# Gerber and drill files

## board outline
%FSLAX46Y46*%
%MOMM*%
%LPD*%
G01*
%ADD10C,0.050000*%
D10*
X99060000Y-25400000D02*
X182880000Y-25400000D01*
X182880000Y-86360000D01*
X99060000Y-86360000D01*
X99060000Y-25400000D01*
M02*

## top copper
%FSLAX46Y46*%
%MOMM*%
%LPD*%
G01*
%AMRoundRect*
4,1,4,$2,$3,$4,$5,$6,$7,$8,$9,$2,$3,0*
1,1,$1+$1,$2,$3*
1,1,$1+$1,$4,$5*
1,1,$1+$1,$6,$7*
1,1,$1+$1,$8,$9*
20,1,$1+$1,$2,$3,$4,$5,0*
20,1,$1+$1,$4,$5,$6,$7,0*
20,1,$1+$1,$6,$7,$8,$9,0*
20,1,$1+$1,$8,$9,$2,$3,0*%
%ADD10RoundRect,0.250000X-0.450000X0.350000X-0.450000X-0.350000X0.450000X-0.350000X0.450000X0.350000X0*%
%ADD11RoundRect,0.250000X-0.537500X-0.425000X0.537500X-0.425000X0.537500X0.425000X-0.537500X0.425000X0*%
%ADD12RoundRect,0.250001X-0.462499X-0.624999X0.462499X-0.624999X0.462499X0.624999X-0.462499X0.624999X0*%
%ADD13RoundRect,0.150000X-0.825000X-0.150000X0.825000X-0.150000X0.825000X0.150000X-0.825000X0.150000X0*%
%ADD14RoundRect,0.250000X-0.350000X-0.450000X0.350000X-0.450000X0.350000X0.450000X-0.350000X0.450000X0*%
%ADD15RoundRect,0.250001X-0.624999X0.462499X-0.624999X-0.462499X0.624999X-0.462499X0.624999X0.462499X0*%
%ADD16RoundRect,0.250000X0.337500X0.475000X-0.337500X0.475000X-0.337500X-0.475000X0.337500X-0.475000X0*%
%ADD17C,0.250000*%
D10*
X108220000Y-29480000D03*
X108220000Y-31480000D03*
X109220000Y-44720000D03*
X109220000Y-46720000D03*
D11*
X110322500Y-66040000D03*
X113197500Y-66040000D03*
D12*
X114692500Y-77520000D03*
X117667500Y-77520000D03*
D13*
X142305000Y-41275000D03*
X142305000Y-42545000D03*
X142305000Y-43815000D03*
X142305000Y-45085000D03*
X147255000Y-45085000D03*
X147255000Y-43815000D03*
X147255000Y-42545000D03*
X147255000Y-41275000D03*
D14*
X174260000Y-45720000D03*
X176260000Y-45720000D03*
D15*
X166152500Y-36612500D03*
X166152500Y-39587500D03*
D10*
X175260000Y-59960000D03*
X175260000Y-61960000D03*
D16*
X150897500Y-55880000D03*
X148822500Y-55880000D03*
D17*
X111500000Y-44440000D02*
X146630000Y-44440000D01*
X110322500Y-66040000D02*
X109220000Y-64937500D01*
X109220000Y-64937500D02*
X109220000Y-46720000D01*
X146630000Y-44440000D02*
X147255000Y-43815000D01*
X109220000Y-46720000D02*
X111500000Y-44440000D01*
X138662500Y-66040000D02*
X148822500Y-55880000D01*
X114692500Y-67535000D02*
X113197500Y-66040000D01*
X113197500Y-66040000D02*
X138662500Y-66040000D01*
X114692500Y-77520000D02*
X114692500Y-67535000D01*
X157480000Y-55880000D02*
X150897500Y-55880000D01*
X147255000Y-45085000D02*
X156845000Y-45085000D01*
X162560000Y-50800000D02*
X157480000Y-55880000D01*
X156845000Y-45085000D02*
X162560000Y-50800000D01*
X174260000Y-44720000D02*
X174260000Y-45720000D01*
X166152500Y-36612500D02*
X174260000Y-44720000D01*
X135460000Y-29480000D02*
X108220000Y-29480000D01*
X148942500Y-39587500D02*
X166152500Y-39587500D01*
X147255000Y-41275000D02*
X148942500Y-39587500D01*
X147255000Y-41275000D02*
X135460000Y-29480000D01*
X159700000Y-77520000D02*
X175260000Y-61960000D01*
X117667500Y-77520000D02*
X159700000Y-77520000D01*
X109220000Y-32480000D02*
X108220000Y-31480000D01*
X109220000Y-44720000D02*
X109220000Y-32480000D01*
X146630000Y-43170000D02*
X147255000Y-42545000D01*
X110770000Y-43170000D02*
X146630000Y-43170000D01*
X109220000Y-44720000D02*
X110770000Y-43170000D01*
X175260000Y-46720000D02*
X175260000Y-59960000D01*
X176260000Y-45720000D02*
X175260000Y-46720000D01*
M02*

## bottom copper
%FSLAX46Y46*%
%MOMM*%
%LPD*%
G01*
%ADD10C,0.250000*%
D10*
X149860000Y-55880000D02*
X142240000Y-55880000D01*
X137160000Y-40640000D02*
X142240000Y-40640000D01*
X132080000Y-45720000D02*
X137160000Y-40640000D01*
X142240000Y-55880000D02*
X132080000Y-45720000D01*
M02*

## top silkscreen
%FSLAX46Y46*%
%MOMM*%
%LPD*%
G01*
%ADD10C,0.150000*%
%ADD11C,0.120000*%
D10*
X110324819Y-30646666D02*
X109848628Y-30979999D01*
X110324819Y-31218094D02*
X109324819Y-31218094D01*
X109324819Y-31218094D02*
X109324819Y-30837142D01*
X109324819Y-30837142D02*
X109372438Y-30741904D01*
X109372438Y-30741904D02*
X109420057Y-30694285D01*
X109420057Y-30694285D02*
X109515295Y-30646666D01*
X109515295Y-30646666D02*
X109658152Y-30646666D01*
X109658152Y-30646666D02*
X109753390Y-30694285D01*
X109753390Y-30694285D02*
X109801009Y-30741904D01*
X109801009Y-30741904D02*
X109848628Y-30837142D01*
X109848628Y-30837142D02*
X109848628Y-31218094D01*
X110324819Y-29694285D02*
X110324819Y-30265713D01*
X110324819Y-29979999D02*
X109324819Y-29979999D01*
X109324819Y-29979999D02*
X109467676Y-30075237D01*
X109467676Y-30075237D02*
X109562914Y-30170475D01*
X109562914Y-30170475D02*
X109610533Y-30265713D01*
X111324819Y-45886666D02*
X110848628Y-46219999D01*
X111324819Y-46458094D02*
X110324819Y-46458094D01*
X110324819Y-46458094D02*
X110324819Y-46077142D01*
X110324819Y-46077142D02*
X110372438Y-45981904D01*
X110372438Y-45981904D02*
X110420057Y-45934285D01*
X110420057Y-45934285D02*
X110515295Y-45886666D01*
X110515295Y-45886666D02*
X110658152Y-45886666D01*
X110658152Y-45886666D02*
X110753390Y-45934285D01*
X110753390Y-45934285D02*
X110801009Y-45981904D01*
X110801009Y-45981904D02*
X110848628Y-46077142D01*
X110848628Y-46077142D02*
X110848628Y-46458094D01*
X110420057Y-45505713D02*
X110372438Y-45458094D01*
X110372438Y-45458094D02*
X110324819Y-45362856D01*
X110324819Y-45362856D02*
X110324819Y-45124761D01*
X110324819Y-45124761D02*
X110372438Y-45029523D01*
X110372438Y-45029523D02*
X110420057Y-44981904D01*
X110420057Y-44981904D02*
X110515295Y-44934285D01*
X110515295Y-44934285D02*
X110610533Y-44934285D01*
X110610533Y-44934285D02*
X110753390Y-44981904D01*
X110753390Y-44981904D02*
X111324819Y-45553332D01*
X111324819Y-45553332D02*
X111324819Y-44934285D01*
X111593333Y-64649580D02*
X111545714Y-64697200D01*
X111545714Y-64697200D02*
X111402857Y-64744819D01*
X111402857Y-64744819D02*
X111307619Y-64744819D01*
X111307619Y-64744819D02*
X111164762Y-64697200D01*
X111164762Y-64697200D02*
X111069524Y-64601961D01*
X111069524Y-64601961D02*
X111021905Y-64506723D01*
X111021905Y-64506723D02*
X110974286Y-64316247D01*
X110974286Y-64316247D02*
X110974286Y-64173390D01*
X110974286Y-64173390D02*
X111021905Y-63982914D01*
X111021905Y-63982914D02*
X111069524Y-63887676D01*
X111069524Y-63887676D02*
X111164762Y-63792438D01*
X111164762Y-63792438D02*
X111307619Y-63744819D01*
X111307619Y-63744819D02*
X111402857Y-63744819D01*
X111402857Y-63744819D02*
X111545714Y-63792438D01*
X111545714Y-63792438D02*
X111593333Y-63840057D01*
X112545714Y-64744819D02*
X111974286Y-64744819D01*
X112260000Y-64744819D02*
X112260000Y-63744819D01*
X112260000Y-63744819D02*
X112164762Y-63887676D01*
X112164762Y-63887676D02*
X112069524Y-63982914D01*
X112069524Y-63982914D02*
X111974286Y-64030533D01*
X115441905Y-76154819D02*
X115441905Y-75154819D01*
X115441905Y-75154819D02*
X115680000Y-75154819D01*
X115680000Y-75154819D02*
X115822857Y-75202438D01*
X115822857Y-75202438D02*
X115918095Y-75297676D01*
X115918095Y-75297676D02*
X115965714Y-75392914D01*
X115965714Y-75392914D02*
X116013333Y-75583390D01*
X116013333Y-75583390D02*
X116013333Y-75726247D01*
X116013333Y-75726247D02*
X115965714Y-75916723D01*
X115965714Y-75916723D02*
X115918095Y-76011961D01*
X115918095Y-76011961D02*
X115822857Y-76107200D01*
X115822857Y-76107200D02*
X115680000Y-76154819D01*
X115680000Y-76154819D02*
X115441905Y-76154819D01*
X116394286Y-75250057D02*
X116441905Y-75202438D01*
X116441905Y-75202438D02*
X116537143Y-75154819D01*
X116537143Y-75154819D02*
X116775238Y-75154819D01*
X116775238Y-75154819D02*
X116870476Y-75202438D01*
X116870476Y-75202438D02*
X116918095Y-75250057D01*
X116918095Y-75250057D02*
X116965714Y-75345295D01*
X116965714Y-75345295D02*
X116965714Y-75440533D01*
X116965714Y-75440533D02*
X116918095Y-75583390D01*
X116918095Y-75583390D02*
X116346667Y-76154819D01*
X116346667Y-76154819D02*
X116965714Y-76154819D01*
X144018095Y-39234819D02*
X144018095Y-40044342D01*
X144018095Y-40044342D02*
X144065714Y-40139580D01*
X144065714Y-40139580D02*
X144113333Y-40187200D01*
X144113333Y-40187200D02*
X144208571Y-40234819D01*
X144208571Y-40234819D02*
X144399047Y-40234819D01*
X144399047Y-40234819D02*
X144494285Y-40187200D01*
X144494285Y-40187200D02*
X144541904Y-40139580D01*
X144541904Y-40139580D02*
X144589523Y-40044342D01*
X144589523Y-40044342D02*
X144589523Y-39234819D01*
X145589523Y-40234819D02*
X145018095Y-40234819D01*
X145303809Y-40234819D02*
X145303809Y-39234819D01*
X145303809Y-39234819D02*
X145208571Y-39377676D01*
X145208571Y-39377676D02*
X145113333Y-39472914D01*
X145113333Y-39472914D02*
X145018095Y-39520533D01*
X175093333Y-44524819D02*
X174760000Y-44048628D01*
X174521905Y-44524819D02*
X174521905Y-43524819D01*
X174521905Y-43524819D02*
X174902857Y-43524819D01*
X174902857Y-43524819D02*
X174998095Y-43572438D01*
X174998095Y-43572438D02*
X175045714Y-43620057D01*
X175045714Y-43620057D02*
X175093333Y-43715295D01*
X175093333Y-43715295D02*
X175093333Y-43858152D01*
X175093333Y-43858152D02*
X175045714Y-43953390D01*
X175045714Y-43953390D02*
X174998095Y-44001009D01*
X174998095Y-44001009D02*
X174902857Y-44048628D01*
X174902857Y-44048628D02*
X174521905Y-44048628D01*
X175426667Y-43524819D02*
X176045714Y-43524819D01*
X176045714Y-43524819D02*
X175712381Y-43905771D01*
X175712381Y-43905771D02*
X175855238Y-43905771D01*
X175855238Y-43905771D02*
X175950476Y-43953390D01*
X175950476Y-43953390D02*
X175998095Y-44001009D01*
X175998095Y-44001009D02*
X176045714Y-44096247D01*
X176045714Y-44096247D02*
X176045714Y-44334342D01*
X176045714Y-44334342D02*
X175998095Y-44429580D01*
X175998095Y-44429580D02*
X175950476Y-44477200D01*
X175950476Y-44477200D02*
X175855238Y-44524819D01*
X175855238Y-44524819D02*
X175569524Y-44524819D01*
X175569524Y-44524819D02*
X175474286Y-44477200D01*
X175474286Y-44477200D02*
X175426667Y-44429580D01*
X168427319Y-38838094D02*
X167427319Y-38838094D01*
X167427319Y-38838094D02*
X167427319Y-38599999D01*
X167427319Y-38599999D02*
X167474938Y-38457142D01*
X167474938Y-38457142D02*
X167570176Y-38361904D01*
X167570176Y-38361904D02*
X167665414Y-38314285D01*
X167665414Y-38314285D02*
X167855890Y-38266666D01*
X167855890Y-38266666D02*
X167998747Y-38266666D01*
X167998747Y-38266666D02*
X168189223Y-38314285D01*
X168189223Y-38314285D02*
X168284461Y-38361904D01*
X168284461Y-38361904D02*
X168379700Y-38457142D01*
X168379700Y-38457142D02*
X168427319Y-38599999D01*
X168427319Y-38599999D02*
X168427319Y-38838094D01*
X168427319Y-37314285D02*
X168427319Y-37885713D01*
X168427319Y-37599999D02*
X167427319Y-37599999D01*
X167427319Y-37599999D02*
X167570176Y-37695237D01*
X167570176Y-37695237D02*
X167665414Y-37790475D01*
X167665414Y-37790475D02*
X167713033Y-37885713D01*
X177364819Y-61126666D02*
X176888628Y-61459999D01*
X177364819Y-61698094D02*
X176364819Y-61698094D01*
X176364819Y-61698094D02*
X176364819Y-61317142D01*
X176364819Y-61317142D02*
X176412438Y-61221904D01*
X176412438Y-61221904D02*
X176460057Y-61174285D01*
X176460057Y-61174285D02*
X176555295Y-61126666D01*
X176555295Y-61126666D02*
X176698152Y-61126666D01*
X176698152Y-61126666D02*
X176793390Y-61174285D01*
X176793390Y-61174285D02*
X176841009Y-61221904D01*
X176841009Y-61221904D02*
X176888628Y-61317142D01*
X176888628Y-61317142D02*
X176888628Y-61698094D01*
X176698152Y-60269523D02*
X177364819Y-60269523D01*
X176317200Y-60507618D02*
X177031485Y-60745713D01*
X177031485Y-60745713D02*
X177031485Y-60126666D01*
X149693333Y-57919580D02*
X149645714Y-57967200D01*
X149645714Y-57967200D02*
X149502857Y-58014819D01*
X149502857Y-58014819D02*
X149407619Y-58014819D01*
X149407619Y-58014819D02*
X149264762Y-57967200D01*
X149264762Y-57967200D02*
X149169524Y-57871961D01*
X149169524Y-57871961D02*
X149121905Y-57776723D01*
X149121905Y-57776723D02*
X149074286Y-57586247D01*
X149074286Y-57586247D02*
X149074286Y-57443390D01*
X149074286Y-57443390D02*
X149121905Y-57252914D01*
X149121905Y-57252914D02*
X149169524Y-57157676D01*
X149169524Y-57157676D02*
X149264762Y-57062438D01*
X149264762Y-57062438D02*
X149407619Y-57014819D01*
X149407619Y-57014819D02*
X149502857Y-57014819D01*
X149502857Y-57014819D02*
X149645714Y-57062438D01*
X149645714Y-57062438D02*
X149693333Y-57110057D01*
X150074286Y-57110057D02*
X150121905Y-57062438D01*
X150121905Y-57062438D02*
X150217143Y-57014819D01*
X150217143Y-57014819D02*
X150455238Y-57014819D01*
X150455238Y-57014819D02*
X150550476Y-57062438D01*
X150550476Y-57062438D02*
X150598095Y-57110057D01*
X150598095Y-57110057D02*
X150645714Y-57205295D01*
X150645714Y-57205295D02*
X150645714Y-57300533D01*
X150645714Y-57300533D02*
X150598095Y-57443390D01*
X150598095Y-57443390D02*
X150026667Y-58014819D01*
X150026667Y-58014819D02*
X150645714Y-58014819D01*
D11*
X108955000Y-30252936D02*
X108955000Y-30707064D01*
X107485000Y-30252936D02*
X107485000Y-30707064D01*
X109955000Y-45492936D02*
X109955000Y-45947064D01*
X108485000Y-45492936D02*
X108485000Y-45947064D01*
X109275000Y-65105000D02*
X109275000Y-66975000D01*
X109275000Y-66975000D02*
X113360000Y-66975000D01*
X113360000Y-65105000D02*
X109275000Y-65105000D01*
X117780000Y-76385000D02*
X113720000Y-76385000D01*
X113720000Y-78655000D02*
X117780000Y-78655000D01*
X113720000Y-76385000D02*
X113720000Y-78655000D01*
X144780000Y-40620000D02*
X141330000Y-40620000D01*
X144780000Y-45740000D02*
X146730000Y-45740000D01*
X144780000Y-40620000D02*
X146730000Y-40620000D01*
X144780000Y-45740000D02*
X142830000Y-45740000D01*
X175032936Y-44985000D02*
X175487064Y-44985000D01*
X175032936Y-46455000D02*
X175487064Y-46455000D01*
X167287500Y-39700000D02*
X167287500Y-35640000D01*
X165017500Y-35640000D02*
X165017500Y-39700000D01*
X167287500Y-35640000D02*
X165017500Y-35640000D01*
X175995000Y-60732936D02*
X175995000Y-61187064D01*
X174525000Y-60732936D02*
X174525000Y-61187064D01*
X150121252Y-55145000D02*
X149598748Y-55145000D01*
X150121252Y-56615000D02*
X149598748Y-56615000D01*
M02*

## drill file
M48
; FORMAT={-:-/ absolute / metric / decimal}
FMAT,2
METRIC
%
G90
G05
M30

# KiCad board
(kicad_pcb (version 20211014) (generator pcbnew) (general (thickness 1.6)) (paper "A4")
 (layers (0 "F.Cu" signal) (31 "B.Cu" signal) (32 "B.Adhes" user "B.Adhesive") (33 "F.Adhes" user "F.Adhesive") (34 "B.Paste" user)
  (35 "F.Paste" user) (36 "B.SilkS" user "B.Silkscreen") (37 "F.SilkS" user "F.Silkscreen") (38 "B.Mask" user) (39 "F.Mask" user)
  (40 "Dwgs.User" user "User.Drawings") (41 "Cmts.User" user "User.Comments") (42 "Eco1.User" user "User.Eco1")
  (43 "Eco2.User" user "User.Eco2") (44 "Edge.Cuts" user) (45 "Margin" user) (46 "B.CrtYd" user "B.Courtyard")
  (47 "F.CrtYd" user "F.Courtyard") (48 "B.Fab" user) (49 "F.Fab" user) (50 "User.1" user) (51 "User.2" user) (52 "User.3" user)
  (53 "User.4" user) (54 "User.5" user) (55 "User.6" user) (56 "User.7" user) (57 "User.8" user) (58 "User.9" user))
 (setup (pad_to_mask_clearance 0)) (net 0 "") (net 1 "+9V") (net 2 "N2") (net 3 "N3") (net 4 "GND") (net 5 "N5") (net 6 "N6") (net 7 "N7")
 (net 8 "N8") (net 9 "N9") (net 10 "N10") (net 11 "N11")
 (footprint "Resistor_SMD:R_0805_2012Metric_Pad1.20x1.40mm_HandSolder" (layer "F.Cu") (at 108.22 30.48 -90)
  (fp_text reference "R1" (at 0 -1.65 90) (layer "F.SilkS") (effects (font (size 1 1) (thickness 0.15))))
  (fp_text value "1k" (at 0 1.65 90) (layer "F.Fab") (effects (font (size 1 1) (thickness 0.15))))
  (fp_line (start -0.227064 -0.735) (end 0.227064 -0.735) (layer "F.SilkS") (width 0.12))
  (fp_line (start -0.227064 0.735) (end 0.227064 0.735) (layer "F.SilkS") (width 0.12))
  (pad "1" smd roundrect (at -1 0 270) (size 1.2 1.4) (layers "F.Cu" "F.Paste" "F.Mask") (roundrect_rratio 0.208333) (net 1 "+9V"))
  (pad "2" smd roundrect (at 1 0 270) (size 1.2 1.4) (layers "F.Cu" "F.Paste" "F.Mask") (roundrect_rratio 0.208333) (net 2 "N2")))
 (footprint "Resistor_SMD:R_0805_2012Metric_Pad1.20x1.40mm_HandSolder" (layer "F.Cu") (at 109.22 45.72 -90)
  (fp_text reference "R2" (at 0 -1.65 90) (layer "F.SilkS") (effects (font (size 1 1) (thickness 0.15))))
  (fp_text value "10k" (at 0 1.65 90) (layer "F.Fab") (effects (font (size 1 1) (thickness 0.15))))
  (fp_line (start -0.227064 -0.735) (end 0.227064 -0.735) (layer "F.SilkS") (width 0.12))
  (fp_line (start -0.227064 0.735) (end 0.227064 0.735) (layer "F.SilkS") (width 0.12))
  (pad "1" smd roundrect (at -1 0 270) (size 1.2 1.4) (layers "F.Cu" "F.Paste" "F.Mask") (roundrect_rratio 0.208333) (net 2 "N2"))
  (pad "2" smd roundrect (at 1 0 270) (size 1.2 1.4) (layers "F.Cu" "F.Paste" "F.Mask") (roundrect_rratio 0.208333) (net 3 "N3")))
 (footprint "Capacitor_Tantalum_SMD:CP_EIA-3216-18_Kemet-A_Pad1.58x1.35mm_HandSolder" (layer "F.Cu") (at 111.76 66.04)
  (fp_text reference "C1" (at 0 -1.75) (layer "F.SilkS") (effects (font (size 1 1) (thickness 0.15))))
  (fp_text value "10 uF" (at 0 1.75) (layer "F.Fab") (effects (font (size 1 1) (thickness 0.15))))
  (fp_line (start -2.485 -0.935) (end -2.485 0.935) (layer "F.SilkS") (width 0.12))
  (fp_line (start -2.485 0.935) (end 1.6 0.935) (layer "F.SilkS") (width 0.12))
  (fp_line (start 1.6 -0.935) (end -2.485 -0.935) (layer "F.SilkS") (width 0.12))
  (pad "1" smd roundrect (at -1.4375 0) (size 1.575 1.35) (layers "F.Cu" "F.Paste" "F.Mask") (roundrect_rratio 0.185185) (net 3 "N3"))
  (pad "2" smd roundrect (at 1.4375 0) (size 1.575 1.35) (layers "F.Cu" "F.Paste" "F.Mask") (roundrect_rratio 0.185185) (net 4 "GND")))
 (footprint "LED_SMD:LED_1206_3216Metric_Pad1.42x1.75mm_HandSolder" (layer "F.Cu") (at 116.18 77.52)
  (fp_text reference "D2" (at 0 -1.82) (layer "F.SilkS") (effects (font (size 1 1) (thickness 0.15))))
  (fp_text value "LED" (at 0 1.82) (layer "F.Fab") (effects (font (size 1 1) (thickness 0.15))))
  (fp_line (start 1.6 -1.135) (end -2.46 -1.135) (layer "F.SilkS") (width 0.12))
  (fp_line (start -2.46 1.135) (end 1.6 1.135) (layer "F.SilkS") (width 0.12))
  (fp_line (start -2.46 -1.135) (end -2.46 1.135) (layer "F.SilkS") (width 0.12))
  (pad "1" smd roundrect (at -1.4875 0) (size 1.425 1.75) (layers "F.Cu" "F.Paste" "F.Mask") (roundrect_rratio 0.175439) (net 4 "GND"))
  (pad "2" smd roundrect (at 1.4875 0) (size 1.425 1.75) (layers "F.Cu" "F.Paste" "F.Mask") (roundrect_rratio 0.175439) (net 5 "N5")))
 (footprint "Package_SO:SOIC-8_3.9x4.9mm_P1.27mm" (layer "F.Cu") (at 144.78 43.18)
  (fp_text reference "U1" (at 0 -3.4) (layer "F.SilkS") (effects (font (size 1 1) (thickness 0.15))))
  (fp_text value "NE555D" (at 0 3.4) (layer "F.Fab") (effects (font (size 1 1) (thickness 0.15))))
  (fp_line (start 0 -2.56) (end -3.45 -2.56) (layer "F.SilkS") (width 0.12))
  (fp_line (start 0 2.56) (end 1.95 2.56) (layer "F.SilkS") (width 0.12))
  (fp_line (start 0 -2.56) (end 1.95 -2.56) (layer "F.SilkS") (width 0.12))
  (fp_line (start 0 2.56) (end -1.95 2.56) (layer "F.SilkS") (width 0.12))
  (pad "1" smd roundrect (at -2.475 -1.905) (size 1.95 0.6) (layers "F.Cu" "F.Paste" "F.Mask") (roundrect_rratio 0.25) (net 4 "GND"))
  (pad "2" smd roundrect (at -2.475 -0.635) (size 1.95 0.6) (layers "F.Cu" "F.Paste" "F.Mask") (roundrect_rratio 0.25) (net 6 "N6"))
  (pad "3" smd roundrect (at -2.475 0.635) (size 1.95 0.6) (layers "F.Cu" "F.Paste" "F.Mask") (roundrect_rratio 0.25) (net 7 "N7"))
  (pad "4" smd roundrect (at -2.475 1.905) (size 1.95 0.6) (layers "F.Cu" "F.Paste" "F.Mask") (roundrect_rratio 0.25) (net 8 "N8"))
  (pad "5" smd roundrect (at 2.475 1.905) (size 1.95 0.6) (layers "F.Cu" "F.Paste" "F.Mask") (roundrect_rratio 0.25) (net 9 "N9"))
  (pad "6" smd roundrect (at 2.475 0.635) (size 1.95 0.6) (layers "F.Cu" "F.Paste" "F.Mask") (roundrect_rratio 0.25) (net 3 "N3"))
  (pad "7" smd roundrect (at 2.475 -0.635) (size 1.95 0.6) (layers "F.Cu" "F.Paste" "F.Mask") (roundrect_rratio 0.25) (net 2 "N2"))
  (pad "8" smd roundrect (at 2.475 -1.905) (size 1.95 0.6) (layers "F.Cu" "F.Paste" "F.Mask") (roundrect_rratio 0.25) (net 1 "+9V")))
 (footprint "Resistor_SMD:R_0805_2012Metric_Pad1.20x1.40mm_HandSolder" (layer "F.Cu") (at 175.26 45.72)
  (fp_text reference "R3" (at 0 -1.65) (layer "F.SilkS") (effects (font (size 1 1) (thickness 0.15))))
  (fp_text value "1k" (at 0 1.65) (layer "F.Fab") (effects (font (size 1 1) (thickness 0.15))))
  (fp_line (start -0.227064 -0.735) (end 0.227064 -0.735) (layer "F.SilkS") (width 0.12))
  (fp_line (start -0.227064 0.735) (end 0.227064 0.735) (layer "F.SilkS") (width 0.12))
  (pad "1" smd roundrect (at -1 0) (size 1.2 1.4) (layers "F.Cu" "F.Paste" "F.Mask") (roundrect_rratio 0.208333) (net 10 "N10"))
  (pad "2" smd roundrect (at 1 0) (size 1.2 1.4) (layers "F.Cu" "F.Paste" "F.Mask") (roundrect_rratio 0.208333) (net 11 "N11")))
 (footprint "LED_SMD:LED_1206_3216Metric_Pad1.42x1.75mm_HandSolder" (layer "F.Cu") (at 166.1525 38.1 -90)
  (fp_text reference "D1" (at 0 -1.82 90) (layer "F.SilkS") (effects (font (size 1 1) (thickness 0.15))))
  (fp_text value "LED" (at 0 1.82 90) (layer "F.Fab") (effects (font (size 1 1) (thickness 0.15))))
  (fp_line (start 1.6 -1.135) (end -2.46 -1.135) (layer "F.SilkS") (width 0.12))
  (fp_line (start -2.46 1.135) (end 1.6 1.135) (layer "F.SilkS") (width 0.12))
  (fp_line (start -2.46 -1.135) (end -2.46 1.135) (layer "F.SilkS") (width 0.12))
  (pad "1" smd roundrect (at -1.4875 0 270) (size 1.425 1.75) (layers "F.Cu" "F.Paste" "F.Mask") (roundrect_rratio 0.175439) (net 10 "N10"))
  (pad "2" smd roundrect (at 1.4875 0 270) (size 1.425 1.75) (layers "F.Cu" "F.Paste" "F.Mask") (roundrect_rratio 0.175439) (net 1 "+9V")))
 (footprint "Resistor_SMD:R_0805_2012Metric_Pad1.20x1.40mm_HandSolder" (layer "F.Cu") (at 175.26 60.96 -90)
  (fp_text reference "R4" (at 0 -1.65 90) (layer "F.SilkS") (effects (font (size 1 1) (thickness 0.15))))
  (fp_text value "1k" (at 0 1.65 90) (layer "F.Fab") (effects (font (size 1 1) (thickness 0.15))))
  (fp_line (start -0.227064 -0.735) (end 0.227064 -0.735) (layer "F.SilkS") (width 0.12))
  (fp_line (start -0.227064 0.735) (end 0.227064 0.735) (layer "F.SilkS") (width 0.12))
  (pad "1" smd roundrect (at -1 0 270) (size 1.2 1.4) (layers "F.Cu" "F.Paste" "F.Mask") (roundrect_rratio 0.208333) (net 11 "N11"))
  (pad "2" smd roundrect (at 1 0 270) (size 1.2 1.4) (layers "F.Cu" "F.Paste" "F.Mask") (roundrect_rratio 0.208333) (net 5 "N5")))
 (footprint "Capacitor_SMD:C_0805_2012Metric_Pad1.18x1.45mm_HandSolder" (layer "F.Cu") (at 149.86 55.88 180)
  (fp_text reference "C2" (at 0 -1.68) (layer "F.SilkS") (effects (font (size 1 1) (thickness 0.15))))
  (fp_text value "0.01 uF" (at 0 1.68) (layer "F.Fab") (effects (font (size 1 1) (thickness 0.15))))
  (fp_line (start -0.261252 0.735) (end 0.261252 0.735) (layer "F.SilkS") (width 0.12))
  (fp_line (start -0.261252 -0.735) (end 0.261252 -0.735) (layer "F.SilkS") (width 0.12))
  (pad "1" smd roundrect (at -1.0375 0 180) (size 1.175 1.45) (layers "F.Cu" "F.Paste" "F.Mask") (roundrect_rratio 0.212766) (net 9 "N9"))
  (pad "2" smd roundrect (at 1.0375 0 180) (size 1.175 1.45) (layers "F.Cu" "F.Paste" "F.Mask") (roundrect_rratio 0.212766) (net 4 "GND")))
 (gr_rect (start 99.06 25.4) (end 182.88 86.36) (layer "Edge.Cuts") (width 0.05) (fill none))
 (segment (start 149.86 55.88) (end 142.24 55.88) (width 0.25) (layer "B.Cu") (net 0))
 (segment (start 137.16 40.64) (end 142.24 40.64) (width 0.25) (layer "B.Cu") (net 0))
 (segment (start 132.08 45.72) (end 137.16 40.64) (width 0.25) (layer "B.Cu") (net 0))
 (segment (start 142.24 55.88) (end 132.08 45.72) (width 0.25) (layer "B.Cu") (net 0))
 (segment (start 111.5 44.44) (end 146.63 44.44) (width 0.25) (layer "F.Cu") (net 3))
 (segment (start 110.3225 66.04) (end 109.22 64.9375) (width 0.25) (layer "F.Cu") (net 3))
 (segment (start 109.22 64.9375) (end 109.22 46.72) (width 0.25) (layer "F.Cu") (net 3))
 (segment (start 146.63 44.44) (end 147.255 43.815) (width 0.25) (layer "F.Cu") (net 3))
 (segment (start 109.22 46.72) (end 111.5 44.44) (width 0.25) (layer "F.Cu") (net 3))
 (segment (start 138.6625 66.04) (end 148.8225 55.88) (width 0.25) (layer "F.Cu") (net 4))
 (segment (start 114.6925 67.535) (end 113.1975 66.04) (width 0.25) (layer "F.Cu") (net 4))
 (segment (start 113.1975 66.04) (end 138.6625 66.04) (width 0.25) (layer "F.Cu") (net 4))
 (segment (start 114.6925 77.52) (end 114.6925 67.535) (width 0.25) (layer "F.Cu") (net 4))
 (segment (start 157.48 55.88) (end 150.8975 55.88) (width 0.25) (layer "F.Cu") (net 9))
 (segment (start 147.255 45.085) (end 156.845 45.085) (width 0.25) (layer "F.Cu") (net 9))
 (segment (start 162.56 50.8) (end 157.48 55.88) (width 0.25) (layer "F.Cu") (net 9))
 (segment (start 156.845 45.085) (end 162.56 50.8) (width 0.25) (layer "F.Cu") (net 9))
 (segment (start 174.26 44.72) (end 174.26 45.72) (width 0.25) (layer "F.Cu") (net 10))
 (segment (start 166.1525 36.6125) (end 174.26 44.72) (width 0.25) (layer "F.Cu") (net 10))
 (segment (start 135.46 29.48) (end 108.22 29.48) (width 0.25) (layer "F.Cu") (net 1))
 (segment (start 148.9425 39.5875) (end 166.1525 39.5875) (width 0.25) (layer "F.Cu") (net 1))
 (segment (start 147.255 41.275) (end 148.9425 39.5875) (width 0.25) (layer "F.Cu") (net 1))
 (segment (start 147.255 41.275) (end 135.46 29.48) (width 0.25) (layer "F.Cu") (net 1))
 (segment (start 159.7 77.52) (end 175.26 61.96) (width 0.25) (layer "F.Cu") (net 5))
 (segment (start 117.6675 77.52) (end 159.7 77.52) (width 0.25) (layer "F.Cu") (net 5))
 (segment (start 109.22 32.48) (end 108.22 31.48) (width 0.25) (layer "F.Cu") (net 2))
 (segment (start 109.22 44.72) (end 109.22 32.48) (width 0.25) (layer "F.Cu") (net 2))
 (segment (start 146.63 43.17) (end 147.255 42.545) (width 0.25) (layer "F.Cu") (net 2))
 (segment (start 110.77 43.17) (end 146.63 43.17) (width 0.25) (layer "F.Cu") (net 2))
 (segment (start 109.22 44.72) (end 110.77 43.17) (width 0.25) (layer "F.Cu") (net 2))
 (segment (start 175.26 46.72) (end 175.26 59.96) (width 0.25) (layer "F.Cu") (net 11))
 (segment (start 176.26 45.72) (end 175.26 46.72) (width 0.25) (layer "F.Cu") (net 11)))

